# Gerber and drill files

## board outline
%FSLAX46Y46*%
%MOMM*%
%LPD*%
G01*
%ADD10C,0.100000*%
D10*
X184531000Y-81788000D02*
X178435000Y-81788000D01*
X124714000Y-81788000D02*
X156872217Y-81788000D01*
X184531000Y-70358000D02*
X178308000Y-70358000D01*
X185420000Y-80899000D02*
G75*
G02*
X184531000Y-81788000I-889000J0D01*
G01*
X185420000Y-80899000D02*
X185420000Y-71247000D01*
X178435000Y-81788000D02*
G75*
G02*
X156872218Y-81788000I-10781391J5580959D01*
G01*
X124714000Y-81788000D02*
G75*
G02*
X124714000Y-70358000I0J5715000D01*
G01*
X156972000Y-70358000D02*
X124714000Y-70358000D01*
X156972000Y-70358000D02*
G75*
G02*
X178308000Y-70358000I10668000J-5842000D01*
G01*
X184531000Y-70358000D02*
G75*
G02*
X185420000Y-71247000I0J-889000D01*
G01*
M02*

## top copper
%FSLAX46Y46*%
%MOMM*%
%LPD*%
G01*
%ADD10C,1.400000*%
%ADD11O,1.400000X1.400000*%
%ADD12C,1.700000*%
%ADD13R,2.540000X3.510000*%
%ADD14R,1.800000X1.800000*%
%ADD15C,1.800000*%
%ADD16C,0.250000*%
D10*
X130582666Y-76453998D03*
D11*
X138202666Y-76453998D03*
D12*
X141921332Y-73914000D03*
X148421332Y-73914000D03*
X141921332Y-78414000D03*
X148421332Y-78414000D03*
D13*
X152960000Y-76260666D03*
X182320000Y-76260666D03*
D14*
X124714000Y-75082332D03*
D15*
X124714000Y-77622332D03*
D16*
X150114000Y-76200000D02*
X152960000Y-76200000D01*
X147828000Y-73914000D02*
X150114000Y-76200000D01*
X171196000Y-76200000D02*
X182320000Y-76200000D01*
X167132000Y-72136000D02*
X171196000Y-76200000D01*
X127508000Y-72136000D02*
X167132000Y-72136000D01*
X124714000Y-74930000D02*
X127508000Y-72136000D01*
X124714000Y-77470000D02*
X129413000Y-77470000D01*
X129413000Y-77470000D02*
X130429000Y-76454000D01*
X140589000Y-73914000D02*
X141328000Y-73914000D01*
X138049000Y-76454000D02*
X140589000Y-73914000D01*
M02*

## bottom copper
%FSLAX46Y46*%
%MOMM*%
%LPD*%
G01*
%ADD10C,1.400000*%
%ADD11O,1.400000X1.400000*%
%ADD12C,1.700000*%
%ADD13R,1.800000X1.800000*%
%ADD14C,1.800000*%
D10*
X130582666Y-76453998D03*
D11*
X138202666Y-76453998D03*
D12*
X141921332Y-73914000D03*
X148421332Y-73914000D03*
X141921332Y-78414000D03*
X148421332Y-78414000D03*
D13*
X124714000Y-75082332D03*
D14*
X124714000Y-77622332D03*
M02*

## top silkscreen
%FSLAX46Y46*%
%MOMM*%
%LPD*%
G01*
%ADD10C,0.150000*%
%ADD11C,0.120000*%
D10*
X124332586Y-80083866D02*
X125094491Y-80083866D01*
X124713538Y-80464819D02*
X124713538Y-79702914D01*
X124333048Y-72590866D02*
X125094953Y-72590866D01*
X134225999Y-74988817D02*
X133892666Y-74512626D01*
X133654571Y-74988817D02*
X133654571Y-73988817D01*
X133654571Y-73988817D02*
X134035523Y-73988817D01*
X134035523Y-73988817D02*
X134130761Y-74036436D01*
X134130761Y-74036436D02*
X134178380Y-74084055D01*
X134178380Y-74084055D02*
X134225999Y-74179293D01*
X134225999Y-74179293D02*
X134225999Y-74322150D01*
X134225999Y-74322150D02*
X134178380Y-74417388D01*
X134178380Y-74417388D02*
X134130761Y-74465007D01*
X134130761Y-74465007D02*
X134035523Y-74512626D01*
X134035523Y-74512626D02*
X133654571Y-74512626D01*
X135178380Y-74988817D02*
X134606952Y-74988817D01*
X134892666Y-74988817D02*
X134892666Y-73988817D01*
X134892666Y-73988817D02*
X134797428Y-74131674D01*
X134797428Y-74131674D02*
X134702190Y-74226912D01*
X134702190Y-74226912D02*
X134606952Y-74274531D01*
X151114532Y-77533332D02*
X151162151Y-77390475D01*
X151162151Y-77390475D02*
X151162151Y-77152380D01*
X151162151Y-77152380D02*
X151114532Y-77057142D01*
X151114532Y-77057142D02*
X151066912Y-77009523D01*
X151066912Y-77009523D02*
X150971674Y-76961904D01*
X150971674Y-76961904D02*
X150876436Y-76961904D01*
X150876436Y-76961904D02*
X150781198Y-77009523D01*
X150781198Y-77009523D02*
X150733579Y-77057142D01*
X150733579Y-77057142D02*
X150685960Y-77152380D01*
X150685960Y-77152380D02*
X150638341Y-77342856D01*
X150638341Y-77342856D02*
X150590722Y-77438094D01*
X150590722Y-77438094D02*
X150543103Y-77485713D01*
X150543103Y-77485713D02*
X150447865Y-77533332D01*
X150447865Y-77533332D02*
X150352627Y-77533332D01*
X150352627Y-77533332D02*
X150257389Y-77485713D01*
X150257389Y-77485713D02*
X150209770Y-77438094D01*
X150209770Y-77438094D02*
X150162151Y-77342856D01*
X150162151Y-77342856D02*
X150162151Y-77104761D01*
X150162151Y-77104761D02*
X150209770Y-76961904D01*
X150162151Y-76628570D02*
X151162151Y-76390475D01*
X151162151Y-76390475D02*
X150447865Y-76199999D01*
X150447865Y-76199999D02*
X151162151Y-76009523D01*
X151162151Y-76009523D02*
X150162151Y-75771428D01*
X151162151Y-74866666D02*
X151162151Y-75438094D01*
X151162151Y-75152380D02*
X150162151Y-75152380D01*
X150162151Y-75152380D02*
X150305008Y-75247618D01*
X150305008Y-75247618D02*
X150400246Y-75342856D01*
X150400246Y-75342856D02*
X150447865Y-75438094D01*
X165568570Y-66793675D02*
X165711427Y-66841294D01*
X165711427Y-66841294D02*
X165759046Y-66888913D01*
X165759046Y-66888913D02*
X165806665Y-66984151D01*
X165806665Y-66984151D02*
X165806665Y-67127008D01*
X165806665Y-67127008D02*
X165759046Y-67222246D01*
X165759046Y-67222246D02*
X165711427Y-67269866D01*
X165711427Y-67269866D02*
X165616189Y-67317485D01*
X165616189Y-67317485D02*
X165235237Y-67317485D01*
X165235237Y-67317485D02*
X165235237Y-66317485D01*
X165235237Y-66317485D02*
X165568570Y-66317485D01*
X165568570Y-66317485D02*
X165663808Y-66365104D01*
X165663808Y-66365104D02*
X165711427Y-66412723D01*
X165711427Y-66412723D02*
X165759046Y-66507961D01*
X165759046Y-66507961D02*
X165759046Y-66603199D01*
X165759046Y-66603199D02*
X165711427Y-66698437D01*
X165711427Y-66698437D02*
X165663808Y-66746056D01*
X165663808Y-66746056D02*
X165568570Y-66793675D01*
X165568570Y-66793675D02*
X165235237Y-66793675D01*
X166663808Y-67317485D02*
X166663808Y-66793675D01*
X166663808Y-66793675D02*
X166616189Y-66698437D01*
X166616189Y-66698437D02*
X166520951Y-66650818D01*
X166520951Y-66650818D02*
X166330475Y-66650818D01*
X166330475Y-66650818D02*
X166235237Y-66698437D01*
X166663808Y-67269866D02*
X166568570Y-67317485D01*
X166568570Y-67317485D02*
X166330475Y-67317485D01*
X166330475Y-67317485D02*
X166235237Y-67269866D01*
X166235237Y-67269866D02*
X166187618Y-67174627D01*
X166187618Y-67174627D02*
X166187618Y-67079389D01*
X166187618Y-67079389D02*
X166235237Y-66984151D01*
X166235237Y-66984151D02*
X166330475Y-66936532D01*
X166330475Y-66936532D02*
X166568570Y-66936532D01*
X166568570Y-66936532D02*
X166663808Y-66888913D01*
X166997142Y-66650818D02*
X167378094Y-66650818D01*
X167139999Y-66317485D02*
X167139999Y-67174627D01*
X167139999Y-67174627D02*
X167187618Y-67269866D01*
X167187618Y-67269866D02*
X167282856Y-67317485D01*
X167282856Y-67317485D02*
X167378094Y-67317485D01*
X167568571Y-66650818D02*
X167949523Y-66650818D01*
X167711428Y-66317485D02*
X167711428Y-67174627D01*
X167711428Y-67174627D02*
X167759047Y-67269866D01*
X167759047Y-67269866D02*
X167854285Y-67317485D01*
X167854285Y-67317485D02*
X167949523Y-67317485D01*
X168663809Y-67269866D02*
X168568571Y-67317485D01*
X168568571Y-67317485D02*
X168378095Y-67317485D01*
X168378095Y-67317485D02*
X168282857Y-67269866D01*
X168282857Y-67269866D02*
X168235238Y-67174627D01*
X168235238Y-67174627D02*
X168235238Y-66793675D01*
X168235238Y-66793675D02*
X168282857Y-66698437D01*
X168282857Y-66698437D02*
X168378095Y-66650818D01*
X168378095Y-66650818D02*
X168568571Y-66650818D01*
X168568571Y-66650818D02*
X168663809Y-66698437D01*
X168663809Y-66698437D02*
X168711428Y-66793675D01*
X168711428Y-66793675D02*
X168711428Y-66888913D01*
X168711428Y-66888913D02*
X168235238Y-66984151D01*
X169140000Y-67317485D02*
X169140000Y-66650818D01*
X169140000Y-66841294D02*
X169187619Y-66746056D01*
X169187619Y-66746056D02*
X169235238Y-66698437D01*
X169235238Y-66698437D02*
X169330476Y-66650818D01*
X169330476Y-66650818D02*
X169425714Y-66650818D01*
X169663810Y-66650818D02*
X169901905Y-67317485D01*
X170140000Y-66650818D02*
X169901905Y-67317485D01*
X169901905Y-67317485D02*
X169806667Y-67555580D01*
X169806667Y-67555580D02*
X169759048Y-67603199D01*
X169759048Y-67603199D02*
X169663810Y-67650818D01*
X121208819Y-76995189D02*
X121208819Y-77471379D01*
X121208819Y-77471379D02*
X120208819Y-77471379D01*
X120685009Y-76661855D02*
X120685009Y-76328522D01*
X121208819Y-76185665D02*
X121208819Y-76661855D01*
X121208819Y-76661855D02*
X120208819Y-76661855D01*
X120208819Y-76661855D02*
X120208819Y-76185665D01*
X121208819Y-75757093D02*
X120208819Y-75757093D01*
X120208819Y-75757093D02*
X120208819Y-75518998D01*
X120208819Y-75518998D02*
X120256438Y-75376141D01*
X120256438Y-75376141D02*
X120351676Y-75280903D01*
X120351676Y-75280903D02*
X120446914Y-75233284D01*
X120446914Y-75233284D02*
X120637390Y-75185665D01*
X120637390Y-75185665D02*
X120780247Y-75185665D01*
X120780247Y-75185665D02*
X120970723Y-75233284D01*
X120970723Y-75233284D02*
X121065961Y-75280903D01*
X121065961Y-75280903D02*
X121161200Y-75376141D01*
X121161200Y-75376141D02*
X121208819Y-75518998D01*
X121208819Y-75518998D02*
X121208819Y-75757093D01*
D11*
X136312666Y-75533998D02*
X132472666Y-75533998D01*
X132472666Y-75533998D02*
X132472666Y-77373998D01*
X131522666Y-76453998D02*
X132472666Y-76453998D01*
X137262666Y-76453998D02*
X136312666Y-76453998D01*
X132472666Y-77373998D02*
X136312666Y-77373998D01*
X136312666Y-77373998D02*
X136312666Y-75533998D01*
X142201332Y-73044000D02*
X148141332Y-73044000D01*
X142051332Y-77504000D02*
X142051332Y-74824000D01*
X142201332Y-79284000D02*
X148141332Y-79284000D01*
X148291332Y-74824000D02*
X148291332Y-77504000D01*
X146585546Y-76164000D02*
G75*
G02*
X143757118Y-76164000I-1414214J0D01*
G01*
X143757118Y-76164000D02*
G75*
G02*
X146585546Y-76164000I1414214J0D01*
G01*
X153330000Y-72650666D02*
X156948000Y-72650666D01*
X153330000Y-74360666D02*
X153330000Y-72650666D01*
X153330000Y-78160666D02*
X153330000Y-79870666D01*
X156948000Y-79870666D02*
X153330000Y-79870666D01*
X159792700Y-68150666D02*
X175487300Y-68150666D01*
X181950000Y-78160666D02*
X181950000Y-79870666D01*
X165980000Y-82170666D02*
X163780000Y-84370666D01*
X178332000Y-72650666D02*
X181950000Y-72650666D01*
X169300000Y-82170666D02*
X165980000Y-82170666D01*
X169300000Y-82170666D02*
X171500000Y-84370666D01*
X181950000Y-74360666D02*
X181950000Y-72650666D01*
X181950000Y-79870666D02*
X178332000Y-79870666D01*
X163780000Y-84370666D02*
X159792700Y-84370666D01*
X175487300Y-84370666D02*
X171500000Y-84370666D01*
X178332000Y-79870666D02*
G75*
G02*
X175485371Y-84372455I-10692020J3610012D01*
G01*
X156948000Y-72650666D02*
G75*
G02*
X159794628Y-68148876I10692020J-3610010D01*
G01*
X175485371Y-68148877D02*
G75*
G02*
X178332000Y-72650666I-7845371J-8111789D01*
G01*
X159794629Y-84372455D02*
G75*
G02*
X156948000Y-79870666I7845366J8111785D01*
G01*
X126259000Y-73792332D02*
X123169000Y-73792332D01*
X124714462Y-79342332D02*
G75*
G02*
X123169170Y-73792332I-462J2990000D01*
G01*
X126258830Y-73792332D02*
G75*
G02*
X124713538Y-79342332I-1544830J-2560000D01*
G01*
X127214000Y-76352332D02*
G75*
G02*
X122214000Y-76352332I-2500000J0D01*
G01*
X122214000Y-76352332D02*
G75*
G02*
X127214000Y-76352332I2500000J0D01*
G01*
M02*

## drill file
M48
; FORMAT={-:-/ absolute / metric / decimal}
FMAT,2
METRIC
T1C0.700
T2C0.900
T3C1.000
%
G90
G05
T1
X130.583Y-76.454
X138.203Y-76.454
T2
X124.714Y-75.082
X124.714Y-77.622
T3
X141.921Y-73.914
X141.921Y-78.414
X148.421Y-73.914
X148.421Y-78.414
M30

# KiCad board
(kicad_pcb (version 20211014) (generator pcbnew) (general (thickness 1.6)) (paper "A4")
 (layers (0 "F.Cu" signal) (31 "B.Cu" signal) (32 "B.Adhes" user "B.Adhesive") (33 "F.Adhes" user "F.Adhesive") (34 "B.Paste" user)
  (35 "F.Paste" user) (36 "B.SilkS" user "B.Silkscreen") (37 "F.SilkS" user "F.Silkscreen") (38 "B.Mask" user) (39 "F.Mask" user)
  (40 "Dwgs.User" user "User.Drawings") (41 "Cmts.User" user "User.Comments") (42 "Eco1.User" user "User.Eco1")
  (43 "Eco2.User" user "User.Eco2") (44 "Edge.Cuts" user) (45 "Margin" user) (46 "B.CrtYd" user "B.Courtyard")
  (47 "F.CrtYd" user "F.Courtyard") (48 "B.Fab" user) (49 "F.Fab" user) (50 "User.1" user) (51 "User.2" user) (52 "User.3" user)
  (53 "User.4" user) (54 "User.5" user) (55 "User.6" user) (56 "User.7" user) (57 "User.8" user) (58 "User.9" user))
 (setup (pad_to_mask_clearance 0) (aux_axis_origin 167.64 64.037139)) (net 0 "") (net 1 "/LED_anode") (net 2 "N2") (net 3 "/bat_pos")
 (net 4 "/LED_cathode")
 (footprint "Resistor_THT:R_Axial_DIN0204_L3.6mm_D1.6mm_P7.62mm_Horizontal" (layer "F.Cu") (at 130.582666 76.453998)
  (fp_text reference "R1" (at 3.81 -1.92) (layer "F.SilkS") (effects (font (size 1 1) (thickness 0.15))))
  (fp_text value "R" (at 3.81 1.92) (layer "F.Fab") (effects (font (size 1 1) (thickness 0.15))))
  (fp_line (start 5.73 -0.92) (end 1.89 -0.92) (layer "F.SilkS") (width 0.12))
  (fp_line (start 1.89 -0.92) (end 1.89 0.92) (layer "F.SilkS") (width 0.12))
  (fp_line (start 0.94 0) (end 1.89 0) (layer "F.SilkS") (width 0.12))
  (fp_line (start 6.68 0) (end 5.73 0) (layer "F.SilkS") (width 0.12))
  (fp_line (start 1.89 0.92) (end 5.73 0.92) (layer "F.SilkS") (width 0.12))
  (fp_line (start 5.73 0.92) (end 5.73 -0.92) (layer "F.SilkS") (width 0.12))
  (pad "1" thru_hole circle (at 0 0) (size 1.4 1.4) (drill 0.7) (layers *.Cu *.Mask) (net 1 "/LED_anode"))
  (pad "2" thru_hole oval (at 7.62 0) (size 1.4 1.4) (drill 0.7) (layers *.Cu *.Mask) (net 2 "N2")))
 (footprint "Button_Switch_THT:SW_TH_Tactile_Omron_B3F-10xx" (layer "F.Cu") (at 141.921332 73.914)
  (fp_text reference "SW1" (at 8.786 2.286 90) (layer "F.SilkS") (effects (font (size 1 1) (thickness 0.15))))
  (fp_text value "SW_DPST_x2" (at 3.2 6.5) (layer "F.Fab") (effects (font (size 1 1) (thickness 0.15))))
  (fp_line (start 0.28 -0.87) (end 6.22 -0.87) (layer "F.SilkS") (width 0.12))
  (fp_line (start 0.13 3.59) (end 0.13 0.91) (layer "F.SilkS") (width 0.12))
  (fp_line (start 0.28 5.37) (end 6.22 5.37) (layer "F.SilkS") (width 0.12))
  (fp_line (start 6.37 0.91) (end 6.37 3.59) (layer "F.SilkS") (width 0.12))
  (fp_circle (center 3.25 2.25) (end 4.25 3.25) (layer "F.SilkS") (width 0.12) (fill none))
  (pad "1" thru_hole circle (at 0 0) (size 1.7 1.7) (drill 1) (layers *.Cu *.Mask) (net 2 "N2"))
  (pad "2" thru_hole circle (at 6.5 0) (size 1.7 1.7) (drill 1) (layers *.Cu *.Mask) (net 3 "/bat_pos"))
  (pad "3" thru_hole circle (at 0 4.5) (size 1.7 1.7) (drill 1) (layers *.Cu *.Mask))
  (pad "4" thru_hole circle (at 6.5 4.5) (size 1.7 1.7) (drill 1) (layers *.Cu *.Mask)))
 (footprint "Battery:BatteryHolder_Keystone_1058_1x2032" (layer "F.Cu") (at 167.64 76.260666)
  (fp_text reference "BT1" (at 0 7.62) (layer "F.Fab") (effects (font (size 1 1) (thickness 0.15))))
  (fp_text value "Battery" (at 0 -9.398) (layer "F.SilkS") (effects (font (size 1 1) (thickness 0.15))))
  (fp_line (start -14.31 -3.61) (end -10.692 -3.61) (layer "F.SilkS") (width 0.12))
  (fp_line (start -14.31 -1.9) (end -14.31 -3.61) (layer "F.SilkS") (width 0.12))
  (fp_line (start -14.31 1.9) (end -14.31 3.61) (layer "F.SilkS") (width 0.12))
  (fp_line (start -10.692 3.61) (end -14.31 3.61) (layer "F.SilkS") (width 0.12))
  (fp_line (start -7.8473 -8.11) (end 7.8473 -8.11) (layer "F.SilkS") (width 0.12))
  (fp_line (start 14.31 1.9) (end 14.31 3.61) (layer "F.SilkS") (width 0.12))
  (fp_line (start -1.66 5.91) (end -3.86 8.11) (layer "F.SilkS") (width 0.12))
  (fp_line (start 10.692 -3.61) (end 14.31 -3.61) (layer "F.SilkS") (width 0.12))
  (fp_line (start 1.66 5.91) (end -1.66 5.91) (layer "F.SilkS") (width 0.12))
  (fp_line (start 1.66 5.91) (end 3.86 8.11) (layer "F.SilkS") (width 0.12))
  (fp_line (start 14.31 -1.9) (end 14.31 -3.61) (layer "F.SilkS") (width 0.12))
  (fp_line (start 14.31 3.61) (end 10.692 3.61) (layer "F.SilkS") (width 0.12))
  (fp_line (start -3.86 8.11) (end -7.8473 8.11) (layer "F.SilkS") (width 0.12))
  (fp_line (start 7.8473 8.11) (end 3.86 8.11) (layer "F.SilkS") (width 0.12))
  (fp_arc (start 10.692 3.61) (mid 9.538084 6.031244) (end 7.845371 8.111789) (layer "F.SilkS") (width 0.12))
  (fp_arc (start -10.692 -3.61) (mid -9.538084 -6.031244) (end -7.845371 -8.111789) (layer "F.SilkS") (width 0.12))
  (fp_arc (start 7.845371 -8.111789) (mid 9.538085 -6.031244) (end 10.692 -3.61) (layer "F.SilkS") (width 0.12))
  (fp_arc (start -7.845371 8.111789) (mid -9.538085 6.031244) (end -10.692 3.61) (layer "F.SilkS") (width 0.12))
  (pad "1" smd rect (at -14.68 0) (size 2.54 3.51) (layers "F.Cu" "F.Paste" "F.Mask") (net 3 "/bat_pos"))
  (pad "2" smd rect (at 14.68 0) (size 2.54 3.51) (layers "F.Cu" "F.Paste" "F.Mask") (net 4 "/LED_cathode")))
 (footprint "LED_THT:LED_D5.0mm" (layer "F.Cu") (at 124.714 75.082332 -90)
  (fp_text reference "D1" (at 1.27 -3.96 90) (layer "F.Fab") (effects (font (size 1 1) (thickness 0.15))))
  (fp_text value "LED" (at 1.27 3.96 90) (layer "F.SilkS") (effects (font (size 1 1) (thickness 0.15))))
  (fp_line (start -1.29 -1.545) (end -1.29 1.545) (layer "F.SilkS") (width 0.12))
  (fp_arc (start 4.26 -0.000462) (mid 2.072002 2.880433) (end -1.29 1.54483) (layer "F.SilkS") (width 0.12))
  (fp_arc (start -1.29 -1.54483) (mid 2.072002 -2.880433) (end 4.26 0.000462) (layer "F.SilkS") (width 0.12))
  (fp_circle (center 1.27 0) (end 3.77 0) (layer "F.SilkS") (width 0.12) (fill none))
  (pad "1" thru_hole rect (at 0 0 270) (size 1.8 1.8) (drill 0.9) (layers *.Cu *.Mask) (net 4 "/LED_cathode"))
  (pad "2" thru_hole circle (at 2.54 0 270) (size 1.8 1.8) (drill 0.9) (layers *.Cu *.Mask) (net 1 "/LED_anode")))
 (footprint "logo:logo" (layer "B.Cu") (at 167.64 76.073 180)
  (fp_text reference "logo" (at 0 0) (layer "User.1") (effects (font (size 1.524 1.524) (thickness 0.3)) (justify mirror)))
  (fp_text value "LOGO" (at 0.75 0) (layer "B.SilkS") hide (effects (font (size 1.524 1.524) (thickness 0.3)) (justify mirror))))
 (gr_line (start 184.531 81.788) (end 178.435 81.788) (layer "Edge.Cuts") (width 0.1))
 (gr_line (start 124.714 81.788) (end 156.872217 81.788) (layer "Edge.Cuts") (width 0.1))
 (gr_line (start 184.531 70.358) (end 178.308 70.358) (layer "Edge.Cuts") (width 0.1))
 (gr_arc (start 185.42 80.899) (mid 185.159618 81.527618) (end 184.531 81.788) (layer "Edge.Cuts") (width 0.1))
 (gr_line (start 185.42 80.899) (end 185.42 71.247) (layer "Edge.Cuts") (width 0.1))
 (gr_arc (start 178.435 81.788) (mid 167.653609 88.347284) (end 156.872217 81.788) (layer "Edge.Cuts") (width 0.1))
 (gr_arc (start 124.714 81.788) (mid 118.999 76.073) (end 124.714 70.358) (layer "Edge.Cuts") (width 0.1))
 (gr_line (start 156.972 70.358) (end 124.714 70.358) (layer "Edge.Cuts") (width 0.1))
 (gr_arc (start 156.972 70.358) (mid 167.64 64.037139) (end 178.308 70.358) (layer "Edge.Cuts") (width 0.1))
 (gr_arc (start 184.531 70.358) (mid 185.159618 70.618382) (end 185.42 71.247) (layer "Edge.Cuts") (width 0.1))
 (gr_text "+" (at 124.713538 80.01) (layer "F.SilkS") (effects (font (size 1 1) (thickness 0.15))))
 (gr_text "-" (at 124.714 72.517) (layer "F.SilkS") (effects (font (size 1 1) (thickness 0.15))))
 (segment (start 150.114 76.2) (end 152.96 76.2) (width 0.25) (layer "F.Cu") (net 3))
 (segment (start 147.828 73.914) (end 150.114 76.2) (width 0.25) (layer "F.Cu") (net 3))
 (segment (start 171.196 76.2) (end 182.32 76.2) (width 0.25) (layer "F.Cu") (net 4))
 (segment (start 167.132 72.136) (end 171.196 76.2) (width 0.25) (layer "F.Cu") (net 4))
 (segment (start 127.508 72.136) (end 167.132 72.136) (width 0.25) (layer "F.Cu") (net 4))
 (segment (start 124.714 74.93) (end 127.508 72.136) (width 0.25) (layer "F.Cu") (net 4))
 (segment (start 124.714 77.47) (end 129.413 77.47) (width 0.25) (layer "F.Cu") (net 1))
 (segment (start 129.413 77.47) (end 130.429 76.454) (width 0.25) (layer "F.Cu") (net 1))
 (segment (start 140.589 73.914) (end 141.328 73.914) (width 0.25) (layer "F.Cu") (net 2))
 (segment (start 138.049 76.454) (end 140.589 73.914) (width 0.25) (layer "F.Cu") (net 2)))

